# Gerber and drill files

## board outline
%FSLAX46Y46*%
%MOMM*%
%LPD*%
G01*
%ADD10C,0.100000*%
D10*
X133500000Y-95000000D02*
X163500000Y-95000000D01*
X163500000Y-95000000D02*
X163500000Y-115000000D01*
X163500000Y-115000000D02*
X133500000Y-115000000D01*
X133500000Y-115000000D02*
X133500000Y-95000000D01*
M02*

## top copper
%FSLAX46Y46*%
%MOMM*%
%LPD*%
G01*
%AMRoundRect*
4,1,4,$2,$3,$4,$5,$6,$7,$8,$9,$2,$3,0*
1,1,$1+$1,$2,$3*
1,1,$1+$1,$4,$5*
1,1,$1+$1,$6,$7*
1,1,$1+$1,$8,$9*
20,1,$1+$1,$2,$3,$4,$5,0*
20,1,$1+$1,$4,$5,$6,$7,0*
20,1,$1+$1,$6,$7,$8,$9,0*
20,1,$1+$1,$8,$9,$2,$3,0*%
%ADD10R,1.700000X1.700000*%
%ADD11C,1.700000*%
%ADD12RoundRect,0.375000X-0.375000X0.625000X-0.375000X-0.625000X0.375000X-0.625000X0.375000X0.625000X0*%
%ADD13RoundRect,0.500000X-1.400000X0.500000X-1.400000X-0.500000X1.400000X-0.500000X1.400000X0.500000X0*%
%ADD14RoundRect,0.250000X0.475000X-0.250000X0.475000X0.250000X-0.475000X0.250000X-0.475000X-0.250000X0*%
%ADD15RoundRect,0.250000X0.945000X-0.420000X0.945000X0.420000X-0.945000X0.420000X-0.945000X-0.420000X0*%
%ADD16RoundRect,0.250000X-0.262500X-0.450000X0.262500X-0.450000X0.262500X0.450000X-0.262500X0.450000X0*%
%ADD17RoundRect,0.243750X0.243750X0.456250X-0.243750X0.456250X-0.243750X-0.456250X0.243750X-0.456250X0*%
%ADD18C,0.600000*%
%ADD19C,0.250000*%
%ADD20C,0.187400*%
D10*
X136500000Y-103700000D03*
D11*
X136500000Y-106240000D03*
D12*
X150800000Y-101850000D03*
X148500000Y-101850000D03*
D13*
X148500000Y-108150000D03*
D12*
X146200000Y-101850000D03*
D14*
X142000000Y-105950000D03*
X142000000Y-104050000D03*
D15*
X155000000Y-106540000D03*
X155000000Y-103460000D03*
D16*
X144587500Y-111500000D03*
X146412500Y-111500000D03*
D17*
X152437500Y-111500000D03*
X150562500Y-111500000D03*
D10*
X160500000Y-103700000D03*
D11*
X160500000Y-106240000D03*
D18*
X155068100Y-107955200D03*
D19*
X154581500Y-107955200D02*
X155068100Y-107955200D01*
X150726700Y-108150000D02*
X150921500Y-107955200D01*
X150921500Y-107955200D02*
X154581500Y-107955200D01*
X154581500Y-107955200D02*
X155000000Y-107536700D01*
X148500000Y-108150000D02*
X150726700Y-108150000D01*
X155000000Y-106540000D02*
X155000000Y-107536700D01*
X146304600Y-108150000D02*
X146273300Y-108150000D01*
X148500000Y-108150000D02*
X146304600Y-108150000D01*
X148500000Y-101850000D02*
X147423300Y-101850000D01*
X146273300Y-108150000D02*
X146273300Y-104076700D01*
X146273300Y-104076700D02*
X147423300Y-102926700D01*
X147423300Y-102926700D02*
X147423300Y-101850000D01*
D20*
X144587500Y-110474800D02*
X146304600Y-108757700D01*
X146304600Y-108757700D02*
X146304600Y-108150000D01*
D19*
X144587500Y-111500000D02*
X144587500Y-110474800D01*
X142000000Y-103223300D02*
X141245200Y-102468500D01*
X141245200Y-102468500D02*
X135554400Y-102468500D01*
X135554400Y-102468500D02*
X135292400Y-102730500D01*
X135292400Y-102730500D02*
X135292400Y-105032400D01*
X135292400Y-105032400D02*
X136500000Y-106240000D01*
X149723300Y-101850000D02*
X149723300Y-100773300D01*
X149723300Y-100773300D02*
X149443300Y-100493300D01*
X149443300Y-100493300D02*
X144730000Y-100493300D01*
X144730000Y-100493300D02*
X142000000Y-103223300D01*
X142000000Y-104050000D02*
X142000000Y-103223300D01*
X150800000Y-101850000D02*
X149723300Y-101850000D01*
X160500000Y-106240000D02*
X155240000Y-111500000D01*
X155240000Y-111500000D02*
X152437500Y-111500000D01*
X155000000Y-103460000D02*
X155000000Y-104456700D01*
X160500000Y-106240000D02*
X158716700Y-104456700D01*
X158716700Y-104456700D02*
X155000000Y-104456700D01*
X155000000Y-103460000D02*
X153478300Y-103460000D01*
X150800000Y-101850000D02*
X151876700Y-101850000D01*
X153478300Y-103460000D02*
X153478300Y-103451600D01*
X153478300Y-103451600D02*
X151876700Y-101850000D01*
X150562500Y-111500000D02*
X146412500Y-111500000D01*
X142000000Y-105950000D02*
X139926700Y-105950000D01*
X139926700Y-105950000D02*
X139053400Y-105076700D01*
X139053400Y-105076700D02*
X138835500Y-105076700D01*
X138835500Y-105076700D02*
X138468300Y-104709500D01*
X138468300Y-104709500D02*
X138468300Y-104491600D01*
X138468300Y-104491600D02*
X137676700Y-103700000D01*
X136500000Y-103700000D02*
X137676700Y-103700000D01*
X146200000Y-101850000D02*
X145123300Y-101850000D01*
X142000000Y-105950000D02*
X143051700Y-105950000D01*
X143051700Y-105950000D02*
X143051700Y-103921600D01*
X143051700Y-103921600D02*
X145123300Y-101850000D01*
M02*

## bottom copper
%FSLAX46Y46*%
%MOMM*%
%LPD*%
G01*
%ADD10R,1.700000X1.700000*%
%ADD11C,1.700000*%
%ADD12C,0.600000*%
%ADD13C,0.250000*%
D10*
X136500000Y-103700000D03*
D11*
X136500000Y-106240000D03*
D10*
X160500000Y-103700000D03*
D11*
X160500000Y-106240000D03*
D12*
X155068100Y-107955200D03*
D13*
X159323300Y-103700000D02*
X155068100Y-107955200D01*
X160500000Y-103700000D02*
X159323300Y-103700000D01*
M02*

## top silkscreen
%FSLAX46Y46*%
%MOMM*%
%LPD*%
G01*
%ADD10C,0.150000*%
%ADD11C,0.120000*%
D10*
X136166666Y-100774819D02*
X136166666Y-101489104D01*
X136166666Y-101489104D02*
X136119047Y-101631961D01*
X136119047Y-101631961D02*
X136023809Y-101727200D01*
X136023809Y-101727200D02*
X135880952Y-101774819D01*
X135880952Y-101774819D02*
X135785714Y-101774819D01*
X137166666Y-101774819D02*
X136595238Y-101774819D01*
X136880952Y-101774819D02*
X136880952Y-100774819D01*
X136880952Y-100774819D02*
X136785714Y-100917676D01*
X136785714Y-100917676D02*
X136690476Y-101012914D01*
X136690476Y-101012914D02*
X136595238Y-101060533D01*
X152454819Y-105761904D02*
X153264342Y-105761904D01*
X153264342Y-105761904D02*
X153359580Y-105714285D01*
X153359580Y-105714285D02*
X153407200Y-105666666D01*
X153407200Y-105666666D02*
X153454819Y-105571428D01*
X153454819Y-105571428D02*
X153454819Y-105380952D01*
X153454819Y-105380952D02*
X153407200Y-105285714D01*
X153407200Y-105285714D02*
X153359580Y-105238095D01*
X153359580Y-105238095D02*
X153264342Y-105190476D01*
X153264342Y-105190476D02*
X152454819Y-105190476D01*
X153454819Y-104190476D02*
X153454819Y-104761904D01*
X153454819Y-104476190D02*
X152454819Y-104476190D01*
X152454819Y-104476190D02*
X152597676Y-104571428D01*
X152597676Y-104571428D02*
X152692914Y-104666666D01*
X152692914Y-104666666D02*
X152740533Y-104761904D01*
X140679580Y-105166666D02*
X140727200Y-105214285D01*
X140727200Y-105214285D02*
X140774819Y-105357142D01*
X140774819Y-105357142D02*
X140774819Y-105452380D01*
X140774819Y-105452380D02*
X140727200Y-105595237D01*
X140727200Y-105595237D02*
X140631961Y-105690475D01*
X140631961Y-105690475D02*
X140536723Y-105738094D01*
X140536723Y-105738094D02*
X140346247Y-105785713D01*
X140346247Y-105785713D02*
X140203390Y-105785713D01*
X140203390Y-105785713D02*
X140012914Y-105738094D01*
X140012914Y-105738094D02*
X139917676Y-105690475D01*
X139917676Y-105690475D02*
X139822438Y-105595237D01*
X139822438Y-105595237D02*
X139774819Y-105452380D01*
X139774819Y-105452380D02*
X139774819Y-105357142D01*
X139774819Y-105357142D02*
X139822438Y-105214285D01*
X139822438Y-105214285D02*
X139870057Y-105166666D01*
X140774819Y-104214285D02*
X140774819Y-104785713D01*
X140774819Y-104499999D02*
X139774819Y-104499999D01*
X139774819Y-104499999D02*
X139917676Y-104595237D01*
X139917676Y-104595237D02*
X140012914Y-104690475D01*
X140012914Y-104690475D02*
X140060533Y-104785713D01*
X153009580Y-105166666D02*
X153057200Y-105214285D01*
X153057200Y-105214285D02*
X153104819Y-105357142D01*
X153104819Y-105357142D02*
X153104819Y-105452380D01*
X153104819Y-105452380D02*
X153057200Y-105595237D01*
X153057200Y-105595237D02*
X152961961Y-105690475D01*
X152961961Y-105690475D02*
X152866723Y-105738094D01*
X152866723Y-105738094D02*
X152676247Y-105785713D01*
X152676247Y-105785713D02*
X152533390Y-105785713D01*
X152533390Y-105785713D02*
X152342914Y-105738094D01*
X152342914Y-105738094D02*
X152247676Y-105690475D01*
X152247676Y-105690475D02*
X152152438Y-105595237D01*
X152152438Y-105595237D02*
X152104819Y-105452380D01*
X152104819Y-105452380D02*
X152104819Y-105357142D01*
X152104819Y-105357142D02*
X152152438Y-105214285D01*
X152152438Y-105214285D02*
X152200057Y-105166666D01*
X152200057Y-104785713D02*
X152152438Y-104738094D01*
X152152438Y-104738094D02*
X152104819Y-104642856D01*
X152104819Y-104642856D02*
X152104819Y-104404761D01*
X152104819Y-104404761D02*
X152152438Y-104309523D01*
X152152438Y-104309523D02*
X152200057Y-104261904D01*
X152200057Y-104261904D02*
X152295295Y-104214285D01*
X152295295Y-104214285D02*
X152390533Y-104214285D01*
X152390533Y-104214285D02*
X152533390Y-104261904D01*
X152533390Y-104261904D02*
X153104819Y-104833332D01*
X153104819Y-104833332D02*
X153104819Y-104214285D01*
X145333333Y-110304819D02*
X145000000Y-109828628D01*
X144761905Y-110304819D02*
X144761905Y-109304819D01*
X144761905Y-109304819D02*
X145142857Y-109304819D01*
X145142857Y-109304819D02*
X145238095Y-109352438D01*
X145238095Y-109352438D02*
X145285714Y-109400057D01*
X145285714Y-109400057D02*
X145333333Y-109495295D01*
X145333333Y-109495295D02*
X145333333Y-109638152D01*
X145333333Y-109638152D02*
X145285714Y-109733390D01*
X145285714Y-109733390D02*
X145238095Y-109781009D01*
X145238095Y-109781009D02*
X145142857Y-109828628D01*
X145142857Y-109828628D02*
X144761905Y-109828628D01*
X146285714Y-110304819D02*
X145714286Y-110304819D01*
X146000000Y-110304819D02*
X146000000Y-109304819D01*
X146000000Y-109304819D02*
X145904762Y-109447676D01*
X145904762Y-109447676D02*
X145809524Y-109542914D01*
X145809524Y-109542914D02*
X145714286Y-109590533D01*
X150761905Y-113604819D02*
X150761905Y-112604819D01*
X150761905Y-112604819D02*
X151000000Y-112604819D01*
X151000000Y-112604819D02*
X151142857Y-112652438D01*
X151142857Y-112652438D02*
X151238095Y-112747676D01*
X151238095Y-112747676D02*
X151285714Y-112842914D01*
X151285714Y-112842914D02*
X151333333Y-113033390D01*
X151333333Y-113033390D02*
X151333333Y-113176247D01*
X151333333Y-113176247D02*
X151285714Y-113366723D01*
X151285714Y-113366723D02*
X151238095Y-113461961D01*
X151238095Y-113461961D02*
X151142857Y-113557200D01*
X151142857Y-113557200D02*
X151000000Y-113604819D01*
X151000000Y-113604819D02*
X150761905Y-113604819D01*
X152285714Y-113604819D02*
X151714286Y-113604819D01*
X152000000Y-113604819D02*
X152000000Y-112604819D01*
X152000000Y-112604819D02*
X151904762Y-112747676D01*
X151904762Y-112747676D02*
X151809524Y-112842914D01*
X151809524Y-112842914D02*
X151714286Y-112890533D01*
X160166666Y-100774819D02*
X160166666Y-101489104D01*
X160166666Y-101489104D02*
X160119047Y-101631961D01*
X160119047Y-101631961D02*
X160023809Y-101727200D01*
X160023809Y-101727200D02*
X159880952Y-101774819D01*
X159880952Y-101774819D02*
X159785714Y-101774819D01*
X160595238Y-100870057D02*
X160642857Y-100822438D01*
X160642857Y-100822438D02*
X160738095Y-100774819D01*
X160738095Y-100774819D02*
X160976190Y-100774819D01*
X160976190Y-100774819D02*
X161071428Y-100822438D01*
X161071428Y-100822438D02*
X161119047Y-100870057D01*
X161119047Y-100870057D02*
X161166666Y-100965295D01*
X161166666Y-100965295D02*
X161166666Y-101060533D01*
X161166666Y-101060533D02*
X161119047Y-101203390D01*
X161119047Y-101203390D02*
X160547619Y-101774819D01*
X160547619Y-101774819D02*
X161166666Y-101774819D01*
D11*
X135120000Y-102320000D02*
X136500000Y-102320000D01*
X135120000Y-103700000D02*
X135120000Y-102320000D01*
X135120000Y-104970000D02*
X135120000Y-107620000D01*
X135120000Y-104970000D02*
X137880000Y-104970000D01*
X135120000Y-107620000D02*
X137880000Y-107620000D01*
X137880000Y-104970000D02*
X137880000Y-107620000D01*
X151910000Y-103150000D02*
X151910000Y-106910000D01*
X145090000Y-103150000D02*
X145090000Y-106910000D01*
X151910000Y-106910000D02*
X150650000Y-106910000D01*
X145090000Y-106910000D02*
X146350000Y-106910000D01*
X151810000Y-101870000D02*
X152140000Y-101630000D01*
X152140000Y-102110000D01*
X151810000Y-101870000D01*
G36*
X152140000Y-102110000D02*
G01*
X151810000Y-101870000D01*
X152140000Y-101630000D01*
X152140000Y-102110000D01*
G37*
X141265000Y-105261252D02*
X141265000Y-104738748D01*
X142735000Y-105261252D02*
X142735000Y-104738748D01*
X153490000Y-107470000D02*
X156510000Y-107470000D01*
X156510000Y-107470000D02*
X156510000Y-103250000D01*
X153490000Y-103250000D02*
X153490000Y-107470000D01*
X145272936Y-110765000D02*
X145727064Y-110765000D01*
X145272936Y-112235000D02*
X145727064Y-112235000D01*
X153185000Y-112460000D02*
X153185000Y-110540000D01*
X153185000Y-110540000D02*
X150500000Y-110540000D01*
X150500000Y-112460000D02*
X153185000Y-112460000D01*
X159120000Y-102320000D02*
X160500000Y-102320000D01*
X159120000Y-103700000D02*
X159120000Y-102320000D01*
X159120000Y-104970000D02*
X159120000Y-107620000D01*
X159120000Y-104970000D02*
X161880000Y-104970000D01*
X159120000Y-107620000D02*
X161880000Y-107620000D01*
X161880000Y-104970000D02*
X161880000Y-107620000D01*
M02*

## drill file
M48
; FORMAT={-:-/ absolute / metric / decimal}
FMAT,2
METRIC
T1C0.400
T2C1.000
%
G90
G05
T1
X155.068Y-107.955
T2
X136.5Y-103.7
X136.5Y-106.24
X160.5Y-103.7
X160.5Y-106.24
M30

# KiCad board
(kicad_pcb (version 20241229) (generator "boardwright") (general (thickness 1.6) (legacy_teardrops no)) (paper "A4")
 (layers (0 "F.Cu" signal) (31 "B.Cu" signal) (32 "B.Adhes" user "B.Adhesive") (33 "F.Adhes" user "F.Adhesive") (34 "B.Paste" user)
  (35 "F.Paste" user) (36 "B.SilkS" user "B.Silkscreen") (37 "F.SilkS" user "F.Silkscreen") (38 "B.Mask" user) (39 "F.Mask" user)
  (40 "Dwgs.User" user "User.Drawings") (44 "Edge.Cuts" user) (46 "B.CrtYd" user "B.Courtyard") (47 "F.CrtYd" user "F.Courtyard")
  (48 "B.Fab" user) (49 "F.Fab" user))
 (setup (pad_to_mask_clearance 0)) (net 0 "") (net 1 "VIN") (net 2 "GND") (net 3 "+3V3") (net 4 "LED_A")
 (gr_line (start 133.5 95) (end 163.5 95) (stroke (width 0.1) (type default)) (layer "Edge.Cuts"))
 (gr_line (start 163.5 95) (end 163.5 115) (stroke (width 0.1) (type default)) (layer "Edge.Cuts"))
 (gr_line (start 163.5 115) (end 133.5 115) (stroke (width 0.1) (type default)) (layer "Edge.Cuts"))
 (gr_line (start 133.5 115) (end 133.5 95) (stroke (width 0.1) (type default)) (layer "Edge.Cuts"))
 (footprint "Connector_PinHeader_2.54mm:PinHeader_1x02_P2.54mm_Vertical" (layer "F.Cu") (at 136.5 103.7)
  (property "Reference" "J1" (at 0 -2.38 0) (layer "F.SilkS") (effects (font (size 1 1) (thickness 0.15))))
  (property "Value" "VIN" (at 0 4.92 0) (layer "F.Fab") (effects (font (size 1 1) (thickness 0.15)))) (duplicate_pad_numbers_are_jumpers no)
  (fp_line (start -1.38 -1.38) (end 0 -1.38) (stroke (width 0.12) (type solid)) (layer "F.SilkS"))
  (fp_line (start -1.38 0) (end -1.38 -1.38) (stroke (width 0.12) (type solid)) (layer "F.SilkS"))
  (fp_line (start -1.38 1.27) (end -1.38 3.92) (stroke (width 0.12) (type solid)) (layer "F.SilkS"))
  (fp_line (start -1.38 1.27) (end 1.38 1.27) (stroke (width 0.12) (type solid)) (layer "F.SilkS"))
  (fp_line (start -1.38 3.92) (end 1.38 3.92) (stroke (width 0.12) (type solid)) (layer "F.SilkS"))
  (fp_line (start 1.38 1.27) (end 1.38 3.92) (stroke (width 0.12) (type solid)) (layer "F.SilkS"))
  (pad "1" thru_hole rect (at 0 0) (size 1.7 1.7) (drill 1) (layers "*.Cu" "*.Mask") (remove_unused_layers no) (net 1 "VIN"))
  (pad "2" thru_hole circle (at 0 2.54) (size 1.7 1.7) (drill 1) (layers "*.Cu" "*.Mask") (remove_unused_layers no) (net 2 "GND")))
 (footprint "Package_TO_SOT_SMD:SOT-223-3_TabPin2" (layer "F.Cu") (at 148.5 105 -90)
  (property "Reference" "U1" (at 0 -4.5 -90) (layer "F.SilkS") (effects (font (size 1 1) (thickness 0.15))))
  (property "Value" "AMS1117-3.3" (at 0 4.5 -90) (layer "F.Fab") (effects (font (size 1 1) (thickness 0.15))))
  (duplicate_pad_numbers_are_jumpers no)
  (fp_line (start -1.85 -3.41) (end 1.91 -3.41) (stroke (width 0.12) (type solid)) (layer "F.SilkS"))
  (fp_line (start -1.85 3.41) (end 1.91 3.41) (stroke (width 0.12) (type solid)) (layer "F.SilkS"))
  (fp_line (start 1.91 -3.41) (end 1.91 -2.15) (stroke (width 0.12) (type solid)) (layer "F.SilkS"))
  (fp_line (start 1.91 3.41) (end 1.91 2.15) (stroke (width 0.12) (type solid)) (layer "F.SilkS"))
  (fp_poly
   (pts (xy -3.13 -3.31) (xy -3.37 -3.64) (xy -2.89 -3.64) (xy -3.13 -3.31)) (stroke (width 0.12) (type solid)) (fill yes) (layer "F.SilkS"))
  (pad "1" smd roundrect (at -3.15 -2.3 -90) (size 2 1.5) (layers "F.Cu" "F.Mask" "F.Paste") (roundrect_rratio 0.25) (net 2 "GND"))
  (pad "2" smd roundrect (at -3.15 0 -90) (size 2 1.5) (layers "F.Cu" "F.Mask" "F.Paste") (roundrect_rratio 0.25) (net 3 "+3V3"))
  (pad "2" smd roundrect (at 3.15 0 -90) (size 2 3.8) (layers "F.Cu" "F.Mask" "F.Paste") (roundrect_rratio 0.25) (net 3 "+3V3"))
  (pad "3" smd roundrect (at -3.15 2.3 -90) (size 2 1.5) (layers "F.Cu" "F.Mask" "F.Paste") (roundrect_rratio 0.25) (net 1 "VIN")))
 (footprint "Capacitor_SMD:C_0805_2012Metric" (layer "F.Cu") (at 142 105 90)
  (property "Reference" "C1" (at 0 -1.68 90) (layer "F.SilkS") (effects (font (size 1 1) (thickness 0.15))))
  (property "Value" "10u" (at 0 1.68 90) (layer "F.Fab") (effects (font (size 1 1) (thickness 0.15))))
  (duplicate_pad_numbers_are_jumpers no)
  (fp_line (start -0.261252 -0.735) (end 0.261252 -0.735) (stroke (width 0.12) (type solid)) (layer "F.SilkS"))
  (fp_line (start -0.261252 0.735) (end 0.261252 0.735) (stroke (width 0.12) (type solid)) (layer "F.SilkS"))
  (pad "1" smd roundrect (at -0.95 0 90) (size 1 1.45) (layers "F.Cu" "F.Mask" "F.Paste") (roundrect_rratio 0.25) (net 1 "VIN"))
  (pad "2" smd roundrect (at 0.95 0 90) (size 1 1.45) (layers "F.Cu" "F.Mask" "F.Paste") (roundrect_rratio 0.25) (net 2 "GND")))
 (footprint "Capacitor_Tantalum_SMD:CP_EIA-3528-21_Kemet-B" (layer "F.Cu") (at 155 105 90)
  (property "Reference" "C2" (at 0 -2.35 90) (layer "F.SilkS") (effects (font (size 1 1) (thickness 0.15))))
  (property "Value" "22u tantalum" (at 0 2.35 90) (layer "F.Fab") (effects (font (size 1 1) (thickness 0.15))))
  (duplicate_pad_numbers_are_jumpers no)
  (fp_line (start -2.47 -1.51) (end -2.47 1.51) (stroke (width 0.12) (type solid)) (layer "F.SilkS"))
  (fp_line (start -2.47 1.51) (end 1.75 1.51) (stroke (width 0.12) (type solid)) (layer "F.SilkS"))
  (fp_line (start 1.75 -1.51) (end -2.47 -1.51) (stroke (width 0.12) (type solid)) (layer "F.SilkS"))
  (pad "1" smd roundrect (at -1.54 0 90) (size 1.34 2.39) (layers "F.Cu" "F.Mask" "F.Paste") (roundrect_rratio 0.186567) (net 3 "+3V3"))
  (pad "2" smd roundrect (at 1.54 0 90) (size 1.34 2.39) (layers "F.Cu" "F.Mask" "F.Paste") (roundrect_rratio 0.186567) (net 2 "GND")))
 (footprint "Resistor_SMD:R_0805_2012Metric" (layer "F.Cu") (at 145.5 111.5)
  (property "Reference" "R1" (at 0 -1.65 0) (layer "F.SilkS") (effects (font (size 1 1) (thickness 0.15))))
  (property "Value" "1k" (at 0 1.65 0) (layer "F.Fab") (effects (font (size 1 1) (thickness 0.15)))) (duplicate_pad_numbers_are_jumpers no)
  (fp_line (start -0.227064 -0.735) (end 0.227064 -0.735) (stroke (width 0.12) (type solid)) (layer "F.SilkS"))
  (fp_line (start -0.227064 0.735) (end 0.227064 0.735) (stroke (width 0.12) (type solid)) (layer "F.SilkS"))
  (pad "1" smd roundrect (at -0.9125 0) (size 1.025 1.4) (layers "F.Cu" "F.Mask" "F.Paste") (roundrect_rratio 0.243902) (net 3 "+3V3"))
  (pad "2" smd roundrect (at 0.9125 0) (size 1.025 1.4) (layers "F.Cu" "F.Mask" "F.Paste") (roundrect_rratio 0.243902) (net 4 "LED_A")))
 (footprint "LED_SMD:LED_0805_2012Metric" (layer "F.Cu") (at 151.5 111.5 180)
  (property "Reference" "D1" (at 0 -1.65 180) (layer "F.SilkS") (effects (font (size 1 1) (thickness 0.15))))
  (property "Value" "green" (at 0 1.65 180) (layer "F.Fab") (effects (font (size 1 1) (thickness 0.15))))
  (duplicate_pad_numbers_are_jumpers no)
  (fp_line (start -1.685 -0.96) (end -1.685 0.96) (stroke (width 0.12) (type solid)) (layer "F.SilkS"))
  (fp_line (start -1.685 0.96) (end 1 0.96) (stroke (width 0.12) (type solid)) (layer "F.SilkS"))
  (fp_line (start 1 -0.96) (end -1.685 -0.96) (stroke (width 0.12) (type solid)) (layer "F.SilkS"))
  (pad "1" smd roundrect (at -0.9375 0 180) (size 0.975 1.4) (layers "F.Cu" "F.Mask" "F.Paste") (roundrect_rratio 0.25) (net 2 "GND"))
  (pad "2" smd roundrect (at 0.9375 0 180) (size 0.975 1.4) (layers "F.Cu" "F.Mask" "F.Paste") (roundrect_rratio 0.25) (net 4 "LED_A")))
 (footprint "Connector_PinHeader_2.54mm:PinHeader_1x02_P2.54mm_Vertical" (layer "F.Cu") (at 160.5 103.7)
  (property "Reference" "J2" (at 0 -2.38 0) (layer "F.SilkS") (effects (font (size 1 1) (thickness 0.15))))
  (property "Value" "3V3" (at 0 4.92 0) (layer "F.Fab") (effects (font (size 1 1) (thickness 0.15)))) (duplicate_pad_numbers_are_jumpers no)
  (fp_line (start -1.38 -1.38) (end 0 -1.38) (stroke (width 0.12) (type solid)) (layer "F.SilkS"))
  (fp_line (start -1.38 0) (end -1.38 -1.38) (stroke (width 0.12) (type solid)) (layer "F.SilkS"))
  (fp_line (start -1.38 1.27) (end -1.38 3.92) (stroke (width 0.12) (type solid)) (layer "F.SilkS"))
  (fp_line (start -1.38 1.27) (end 1.38 1.27) (stroke (width 0.12) (type solid)) (layer "F.SilkS"))
  (fp_line (start -1.38 3.92) (end 1.38 3.92) (stroke (width 0.12) (type solid)) (layer "F.SilkS"))
  (fp_line (start 1.38 1.27) (end 1.38 3.92) (stroke (width 0.12) (type solid)) (layer "F.SilkS"))
  (pad "1" thru_hole rect (at 0 0) (size 1.7 1.7) (drill 1) (layers "*.Cu" "*.Mask") (remove_unused_layers no) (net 3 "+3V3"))
  (pad "2" thru_hole circle (at 0 2.54) (size 1.7 1.7) (drill 1) (layers "*.Cu" "*.Mask") (remove_unused_layers no) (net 2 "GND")))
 (segment (start 154.5815 107.9552) (end 155.0681 107.9552) (width 0.25) (layer "F.Cu") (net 3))
 (segment (start 150.7267 108.15) (end 150.9215 107.9552) (width 0.25) (layer "F.Cu") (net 3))
 (segment (start 150.9215 107.9552) (end 154.5815 107.9552) (width 0.25) (layer "F.Cu") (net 3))
 (segment (start 154.5815 107.9552) (end 155 107.5367) (width 0.25) (layer "F.Cu") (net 3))
 (segment (start 159.3233 103.7) (end 155.0681 107.9552) (width 0.25) (layer "B.Cu") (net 3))
 (segment (start 160.5 103.7) (end 159.3233 103.7) (width 0.25) (layer "B.Cu") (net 3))
 (segment (start 148.5 108.15) (end 150.7267 108.15) (width 0.25) (layer "F.Cu") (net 3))
 (segment (start 155 106.54) (end 155 107.5367) (width 0.25) (layer "F.Cu") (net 3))
 (segment (start 146.3046 108.15) (end 146.2733 108.15) (width 0.25) (layer "F.Cu") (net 3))
 (segment (start 148.5 108.15) (end 146.3046 108.15) (width 0.25) (layer "F.Cu") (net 3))
 (segment (start 148.5 101.85) (end 147.4233 101.85) (width 0.25) (layer "F.Cu") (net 3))
 (segment (start 146.2733 108.15) (end 146.2733 104.0767) (width 0.25) (layer "F.Cu") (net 3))
 (segment (start 146.2733 104.0767) (end 147.4233 102.9267) (width 0.25) (layer "F.Cu") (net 3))
 (segment (start 147.4233 102.9267) (end 147.4233 101.85) (width 0.25) (layer "F.Cu") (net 3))
 (segment (start 144.5875 110.4748) (end 146.3046 108.7577) (width 0.1874) (layer "F.Cu") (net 3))
 (segment (start 146.3046 108.7577) (end 146.3046 108.15) (width 0.1874) (layer "F.Cu") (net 3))
 (segment (start 144.5875 111.5) (end 144.5875 110.4748) (width 0.25) (layer "F.Cu") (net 3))
 (segment (start 142 103.2233) (end 141.2452 102.4685) (width 0.25) (layer "F.Cu") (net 2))
 (segment (start 141.2452 102.4685) (end 135.5544 102.4685) (width 0.25) (layer "F.Cu") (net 2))
 (segment (start 135.5544 102.4685) (end 135.2924 102.7305) (width 0.25) (layer "F.Cu") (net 2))
 (segment (start 135.2924 102.7305) (end 135.2924 105.0324) (width 0.25) (layer "F.Cu") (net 2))
 (segment (start 135.2924 105.0324) (end 136.5 106.24) (width 0.25) (layer "F.Cu") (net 2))
 (segment (start 149.7233 101.85) (end 149.7233 100.7733) (width 0.25) (layer "F.Cu") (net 2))
 (segment (start 149.7233 100.7733) (end 149.4433 100.4933) (width 0.25) (layer "F.Cu") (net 2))
 (segment (start 149.4433 100.4933) (end 144.73 100.4933) (width 0.25) (layer "F.Cu") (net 2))
 (segment (start 144.73 100.4933) (end 142 103.2233) (width 0.25) (layer "F.Cu") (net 2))
 (segment (start 142 104.05) (end 142 103.2233) (width 0.25) (layer "F.Cu") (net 2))
 (segment (start 150.8 101.85) (end 149.7233 101.85) (width 0.25) (layer "F.Cu") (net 2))
 (segment (start 160.5 106.24) (end 155.24 111.5) (width 0.25) (layer "F.Cu") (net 2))
 (segment (start 155.24 111.5) (end 152.4375 111.5) (width 0.25) (layer "F.Cu") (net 2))
 (segment (start 155 103.46) (end 155 104.4567) (width 0.25) (layer "F.Cu") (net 2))
 (segment (start 160.5 106.24) (end 158.7167 104.4567) (width 0.25) (layer "F.Cu") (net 2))
 (segment (start 158.7167 104.4567) (end 155 104.4567) (width 0.25) (layer "F.Cu") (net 2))
 (segment (start 155 103.46) (end 153.4783 103.46) (width 0.25) (layer "F.Cu") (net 2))
 (segment (start 150.8 101.85) (end 151.8767 101.85) (width 0.25) (layer "F.Cu") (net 2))
 (segment (start 153.4783 103.46) (end 153.4783 103.4516) (width 0.25) (layer "F.Cu") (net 2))
 (segment (start 153.4783 103.4516) (end 151.8767 101.85) (width 0.25) (layer "F.Cu") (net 2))
 (segment (start 150.5625 111.5) (end 146.4125 111.5) (width 0.25) (layer "F.Cu") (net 4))
 (segment (start 142 105.95) (end 139.9267 105.95) (width 0.25) (layer "F.Cu") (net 1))
 (segment (start 139.9267 105.95) (end 139.0534 105.0767) (width 0.25) (layer "F.Cu") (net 1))
 (segment (start 139.0534 105.0767) (end 138.8355 105.0767) (width 0.25) (layer "F.Cu") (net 1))
 (segment (start 138.8355 105.0767) (end 138.4683 104.7095) (width 0.25) (layer "F.Cu") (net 1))
 (segment (start 138.4683 104.7095) (end 138.4683 104.4916) (width 0.25) (layer "F.Cu") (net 1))
 (segment (start 138.4683 104.4916) (end 137.6767 103.7) (width 0.25) (layer "F.Cu") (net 1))
 (segment (start 136.5 103.7) (end 137.6767 103.7) (width 0.25) (layer "F.Cu") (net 1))
 (segment (start 146.2 101.85) (end 145.1233 101.85) (width 0.25) (layer "F.Cu") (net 1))
 (segment (start 142 105.95) (end 143.0517 105.95) (width 0.25) (layer "F.Cu") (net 1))
 (segment (start 143.0517 105.95) (end 143.0517 103.9216) (width 0.25) (layer "F.Cu") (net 1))
 (segment (start 143.0517 103.9216) (end 145.1233 101.85) (width 0.25) (layer "F.Cu") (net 1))
 (via (at 155.0681 107.9552) (size 0.6) (drill 0.4) (layers "F.Cu" "B.Cu") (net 3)))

